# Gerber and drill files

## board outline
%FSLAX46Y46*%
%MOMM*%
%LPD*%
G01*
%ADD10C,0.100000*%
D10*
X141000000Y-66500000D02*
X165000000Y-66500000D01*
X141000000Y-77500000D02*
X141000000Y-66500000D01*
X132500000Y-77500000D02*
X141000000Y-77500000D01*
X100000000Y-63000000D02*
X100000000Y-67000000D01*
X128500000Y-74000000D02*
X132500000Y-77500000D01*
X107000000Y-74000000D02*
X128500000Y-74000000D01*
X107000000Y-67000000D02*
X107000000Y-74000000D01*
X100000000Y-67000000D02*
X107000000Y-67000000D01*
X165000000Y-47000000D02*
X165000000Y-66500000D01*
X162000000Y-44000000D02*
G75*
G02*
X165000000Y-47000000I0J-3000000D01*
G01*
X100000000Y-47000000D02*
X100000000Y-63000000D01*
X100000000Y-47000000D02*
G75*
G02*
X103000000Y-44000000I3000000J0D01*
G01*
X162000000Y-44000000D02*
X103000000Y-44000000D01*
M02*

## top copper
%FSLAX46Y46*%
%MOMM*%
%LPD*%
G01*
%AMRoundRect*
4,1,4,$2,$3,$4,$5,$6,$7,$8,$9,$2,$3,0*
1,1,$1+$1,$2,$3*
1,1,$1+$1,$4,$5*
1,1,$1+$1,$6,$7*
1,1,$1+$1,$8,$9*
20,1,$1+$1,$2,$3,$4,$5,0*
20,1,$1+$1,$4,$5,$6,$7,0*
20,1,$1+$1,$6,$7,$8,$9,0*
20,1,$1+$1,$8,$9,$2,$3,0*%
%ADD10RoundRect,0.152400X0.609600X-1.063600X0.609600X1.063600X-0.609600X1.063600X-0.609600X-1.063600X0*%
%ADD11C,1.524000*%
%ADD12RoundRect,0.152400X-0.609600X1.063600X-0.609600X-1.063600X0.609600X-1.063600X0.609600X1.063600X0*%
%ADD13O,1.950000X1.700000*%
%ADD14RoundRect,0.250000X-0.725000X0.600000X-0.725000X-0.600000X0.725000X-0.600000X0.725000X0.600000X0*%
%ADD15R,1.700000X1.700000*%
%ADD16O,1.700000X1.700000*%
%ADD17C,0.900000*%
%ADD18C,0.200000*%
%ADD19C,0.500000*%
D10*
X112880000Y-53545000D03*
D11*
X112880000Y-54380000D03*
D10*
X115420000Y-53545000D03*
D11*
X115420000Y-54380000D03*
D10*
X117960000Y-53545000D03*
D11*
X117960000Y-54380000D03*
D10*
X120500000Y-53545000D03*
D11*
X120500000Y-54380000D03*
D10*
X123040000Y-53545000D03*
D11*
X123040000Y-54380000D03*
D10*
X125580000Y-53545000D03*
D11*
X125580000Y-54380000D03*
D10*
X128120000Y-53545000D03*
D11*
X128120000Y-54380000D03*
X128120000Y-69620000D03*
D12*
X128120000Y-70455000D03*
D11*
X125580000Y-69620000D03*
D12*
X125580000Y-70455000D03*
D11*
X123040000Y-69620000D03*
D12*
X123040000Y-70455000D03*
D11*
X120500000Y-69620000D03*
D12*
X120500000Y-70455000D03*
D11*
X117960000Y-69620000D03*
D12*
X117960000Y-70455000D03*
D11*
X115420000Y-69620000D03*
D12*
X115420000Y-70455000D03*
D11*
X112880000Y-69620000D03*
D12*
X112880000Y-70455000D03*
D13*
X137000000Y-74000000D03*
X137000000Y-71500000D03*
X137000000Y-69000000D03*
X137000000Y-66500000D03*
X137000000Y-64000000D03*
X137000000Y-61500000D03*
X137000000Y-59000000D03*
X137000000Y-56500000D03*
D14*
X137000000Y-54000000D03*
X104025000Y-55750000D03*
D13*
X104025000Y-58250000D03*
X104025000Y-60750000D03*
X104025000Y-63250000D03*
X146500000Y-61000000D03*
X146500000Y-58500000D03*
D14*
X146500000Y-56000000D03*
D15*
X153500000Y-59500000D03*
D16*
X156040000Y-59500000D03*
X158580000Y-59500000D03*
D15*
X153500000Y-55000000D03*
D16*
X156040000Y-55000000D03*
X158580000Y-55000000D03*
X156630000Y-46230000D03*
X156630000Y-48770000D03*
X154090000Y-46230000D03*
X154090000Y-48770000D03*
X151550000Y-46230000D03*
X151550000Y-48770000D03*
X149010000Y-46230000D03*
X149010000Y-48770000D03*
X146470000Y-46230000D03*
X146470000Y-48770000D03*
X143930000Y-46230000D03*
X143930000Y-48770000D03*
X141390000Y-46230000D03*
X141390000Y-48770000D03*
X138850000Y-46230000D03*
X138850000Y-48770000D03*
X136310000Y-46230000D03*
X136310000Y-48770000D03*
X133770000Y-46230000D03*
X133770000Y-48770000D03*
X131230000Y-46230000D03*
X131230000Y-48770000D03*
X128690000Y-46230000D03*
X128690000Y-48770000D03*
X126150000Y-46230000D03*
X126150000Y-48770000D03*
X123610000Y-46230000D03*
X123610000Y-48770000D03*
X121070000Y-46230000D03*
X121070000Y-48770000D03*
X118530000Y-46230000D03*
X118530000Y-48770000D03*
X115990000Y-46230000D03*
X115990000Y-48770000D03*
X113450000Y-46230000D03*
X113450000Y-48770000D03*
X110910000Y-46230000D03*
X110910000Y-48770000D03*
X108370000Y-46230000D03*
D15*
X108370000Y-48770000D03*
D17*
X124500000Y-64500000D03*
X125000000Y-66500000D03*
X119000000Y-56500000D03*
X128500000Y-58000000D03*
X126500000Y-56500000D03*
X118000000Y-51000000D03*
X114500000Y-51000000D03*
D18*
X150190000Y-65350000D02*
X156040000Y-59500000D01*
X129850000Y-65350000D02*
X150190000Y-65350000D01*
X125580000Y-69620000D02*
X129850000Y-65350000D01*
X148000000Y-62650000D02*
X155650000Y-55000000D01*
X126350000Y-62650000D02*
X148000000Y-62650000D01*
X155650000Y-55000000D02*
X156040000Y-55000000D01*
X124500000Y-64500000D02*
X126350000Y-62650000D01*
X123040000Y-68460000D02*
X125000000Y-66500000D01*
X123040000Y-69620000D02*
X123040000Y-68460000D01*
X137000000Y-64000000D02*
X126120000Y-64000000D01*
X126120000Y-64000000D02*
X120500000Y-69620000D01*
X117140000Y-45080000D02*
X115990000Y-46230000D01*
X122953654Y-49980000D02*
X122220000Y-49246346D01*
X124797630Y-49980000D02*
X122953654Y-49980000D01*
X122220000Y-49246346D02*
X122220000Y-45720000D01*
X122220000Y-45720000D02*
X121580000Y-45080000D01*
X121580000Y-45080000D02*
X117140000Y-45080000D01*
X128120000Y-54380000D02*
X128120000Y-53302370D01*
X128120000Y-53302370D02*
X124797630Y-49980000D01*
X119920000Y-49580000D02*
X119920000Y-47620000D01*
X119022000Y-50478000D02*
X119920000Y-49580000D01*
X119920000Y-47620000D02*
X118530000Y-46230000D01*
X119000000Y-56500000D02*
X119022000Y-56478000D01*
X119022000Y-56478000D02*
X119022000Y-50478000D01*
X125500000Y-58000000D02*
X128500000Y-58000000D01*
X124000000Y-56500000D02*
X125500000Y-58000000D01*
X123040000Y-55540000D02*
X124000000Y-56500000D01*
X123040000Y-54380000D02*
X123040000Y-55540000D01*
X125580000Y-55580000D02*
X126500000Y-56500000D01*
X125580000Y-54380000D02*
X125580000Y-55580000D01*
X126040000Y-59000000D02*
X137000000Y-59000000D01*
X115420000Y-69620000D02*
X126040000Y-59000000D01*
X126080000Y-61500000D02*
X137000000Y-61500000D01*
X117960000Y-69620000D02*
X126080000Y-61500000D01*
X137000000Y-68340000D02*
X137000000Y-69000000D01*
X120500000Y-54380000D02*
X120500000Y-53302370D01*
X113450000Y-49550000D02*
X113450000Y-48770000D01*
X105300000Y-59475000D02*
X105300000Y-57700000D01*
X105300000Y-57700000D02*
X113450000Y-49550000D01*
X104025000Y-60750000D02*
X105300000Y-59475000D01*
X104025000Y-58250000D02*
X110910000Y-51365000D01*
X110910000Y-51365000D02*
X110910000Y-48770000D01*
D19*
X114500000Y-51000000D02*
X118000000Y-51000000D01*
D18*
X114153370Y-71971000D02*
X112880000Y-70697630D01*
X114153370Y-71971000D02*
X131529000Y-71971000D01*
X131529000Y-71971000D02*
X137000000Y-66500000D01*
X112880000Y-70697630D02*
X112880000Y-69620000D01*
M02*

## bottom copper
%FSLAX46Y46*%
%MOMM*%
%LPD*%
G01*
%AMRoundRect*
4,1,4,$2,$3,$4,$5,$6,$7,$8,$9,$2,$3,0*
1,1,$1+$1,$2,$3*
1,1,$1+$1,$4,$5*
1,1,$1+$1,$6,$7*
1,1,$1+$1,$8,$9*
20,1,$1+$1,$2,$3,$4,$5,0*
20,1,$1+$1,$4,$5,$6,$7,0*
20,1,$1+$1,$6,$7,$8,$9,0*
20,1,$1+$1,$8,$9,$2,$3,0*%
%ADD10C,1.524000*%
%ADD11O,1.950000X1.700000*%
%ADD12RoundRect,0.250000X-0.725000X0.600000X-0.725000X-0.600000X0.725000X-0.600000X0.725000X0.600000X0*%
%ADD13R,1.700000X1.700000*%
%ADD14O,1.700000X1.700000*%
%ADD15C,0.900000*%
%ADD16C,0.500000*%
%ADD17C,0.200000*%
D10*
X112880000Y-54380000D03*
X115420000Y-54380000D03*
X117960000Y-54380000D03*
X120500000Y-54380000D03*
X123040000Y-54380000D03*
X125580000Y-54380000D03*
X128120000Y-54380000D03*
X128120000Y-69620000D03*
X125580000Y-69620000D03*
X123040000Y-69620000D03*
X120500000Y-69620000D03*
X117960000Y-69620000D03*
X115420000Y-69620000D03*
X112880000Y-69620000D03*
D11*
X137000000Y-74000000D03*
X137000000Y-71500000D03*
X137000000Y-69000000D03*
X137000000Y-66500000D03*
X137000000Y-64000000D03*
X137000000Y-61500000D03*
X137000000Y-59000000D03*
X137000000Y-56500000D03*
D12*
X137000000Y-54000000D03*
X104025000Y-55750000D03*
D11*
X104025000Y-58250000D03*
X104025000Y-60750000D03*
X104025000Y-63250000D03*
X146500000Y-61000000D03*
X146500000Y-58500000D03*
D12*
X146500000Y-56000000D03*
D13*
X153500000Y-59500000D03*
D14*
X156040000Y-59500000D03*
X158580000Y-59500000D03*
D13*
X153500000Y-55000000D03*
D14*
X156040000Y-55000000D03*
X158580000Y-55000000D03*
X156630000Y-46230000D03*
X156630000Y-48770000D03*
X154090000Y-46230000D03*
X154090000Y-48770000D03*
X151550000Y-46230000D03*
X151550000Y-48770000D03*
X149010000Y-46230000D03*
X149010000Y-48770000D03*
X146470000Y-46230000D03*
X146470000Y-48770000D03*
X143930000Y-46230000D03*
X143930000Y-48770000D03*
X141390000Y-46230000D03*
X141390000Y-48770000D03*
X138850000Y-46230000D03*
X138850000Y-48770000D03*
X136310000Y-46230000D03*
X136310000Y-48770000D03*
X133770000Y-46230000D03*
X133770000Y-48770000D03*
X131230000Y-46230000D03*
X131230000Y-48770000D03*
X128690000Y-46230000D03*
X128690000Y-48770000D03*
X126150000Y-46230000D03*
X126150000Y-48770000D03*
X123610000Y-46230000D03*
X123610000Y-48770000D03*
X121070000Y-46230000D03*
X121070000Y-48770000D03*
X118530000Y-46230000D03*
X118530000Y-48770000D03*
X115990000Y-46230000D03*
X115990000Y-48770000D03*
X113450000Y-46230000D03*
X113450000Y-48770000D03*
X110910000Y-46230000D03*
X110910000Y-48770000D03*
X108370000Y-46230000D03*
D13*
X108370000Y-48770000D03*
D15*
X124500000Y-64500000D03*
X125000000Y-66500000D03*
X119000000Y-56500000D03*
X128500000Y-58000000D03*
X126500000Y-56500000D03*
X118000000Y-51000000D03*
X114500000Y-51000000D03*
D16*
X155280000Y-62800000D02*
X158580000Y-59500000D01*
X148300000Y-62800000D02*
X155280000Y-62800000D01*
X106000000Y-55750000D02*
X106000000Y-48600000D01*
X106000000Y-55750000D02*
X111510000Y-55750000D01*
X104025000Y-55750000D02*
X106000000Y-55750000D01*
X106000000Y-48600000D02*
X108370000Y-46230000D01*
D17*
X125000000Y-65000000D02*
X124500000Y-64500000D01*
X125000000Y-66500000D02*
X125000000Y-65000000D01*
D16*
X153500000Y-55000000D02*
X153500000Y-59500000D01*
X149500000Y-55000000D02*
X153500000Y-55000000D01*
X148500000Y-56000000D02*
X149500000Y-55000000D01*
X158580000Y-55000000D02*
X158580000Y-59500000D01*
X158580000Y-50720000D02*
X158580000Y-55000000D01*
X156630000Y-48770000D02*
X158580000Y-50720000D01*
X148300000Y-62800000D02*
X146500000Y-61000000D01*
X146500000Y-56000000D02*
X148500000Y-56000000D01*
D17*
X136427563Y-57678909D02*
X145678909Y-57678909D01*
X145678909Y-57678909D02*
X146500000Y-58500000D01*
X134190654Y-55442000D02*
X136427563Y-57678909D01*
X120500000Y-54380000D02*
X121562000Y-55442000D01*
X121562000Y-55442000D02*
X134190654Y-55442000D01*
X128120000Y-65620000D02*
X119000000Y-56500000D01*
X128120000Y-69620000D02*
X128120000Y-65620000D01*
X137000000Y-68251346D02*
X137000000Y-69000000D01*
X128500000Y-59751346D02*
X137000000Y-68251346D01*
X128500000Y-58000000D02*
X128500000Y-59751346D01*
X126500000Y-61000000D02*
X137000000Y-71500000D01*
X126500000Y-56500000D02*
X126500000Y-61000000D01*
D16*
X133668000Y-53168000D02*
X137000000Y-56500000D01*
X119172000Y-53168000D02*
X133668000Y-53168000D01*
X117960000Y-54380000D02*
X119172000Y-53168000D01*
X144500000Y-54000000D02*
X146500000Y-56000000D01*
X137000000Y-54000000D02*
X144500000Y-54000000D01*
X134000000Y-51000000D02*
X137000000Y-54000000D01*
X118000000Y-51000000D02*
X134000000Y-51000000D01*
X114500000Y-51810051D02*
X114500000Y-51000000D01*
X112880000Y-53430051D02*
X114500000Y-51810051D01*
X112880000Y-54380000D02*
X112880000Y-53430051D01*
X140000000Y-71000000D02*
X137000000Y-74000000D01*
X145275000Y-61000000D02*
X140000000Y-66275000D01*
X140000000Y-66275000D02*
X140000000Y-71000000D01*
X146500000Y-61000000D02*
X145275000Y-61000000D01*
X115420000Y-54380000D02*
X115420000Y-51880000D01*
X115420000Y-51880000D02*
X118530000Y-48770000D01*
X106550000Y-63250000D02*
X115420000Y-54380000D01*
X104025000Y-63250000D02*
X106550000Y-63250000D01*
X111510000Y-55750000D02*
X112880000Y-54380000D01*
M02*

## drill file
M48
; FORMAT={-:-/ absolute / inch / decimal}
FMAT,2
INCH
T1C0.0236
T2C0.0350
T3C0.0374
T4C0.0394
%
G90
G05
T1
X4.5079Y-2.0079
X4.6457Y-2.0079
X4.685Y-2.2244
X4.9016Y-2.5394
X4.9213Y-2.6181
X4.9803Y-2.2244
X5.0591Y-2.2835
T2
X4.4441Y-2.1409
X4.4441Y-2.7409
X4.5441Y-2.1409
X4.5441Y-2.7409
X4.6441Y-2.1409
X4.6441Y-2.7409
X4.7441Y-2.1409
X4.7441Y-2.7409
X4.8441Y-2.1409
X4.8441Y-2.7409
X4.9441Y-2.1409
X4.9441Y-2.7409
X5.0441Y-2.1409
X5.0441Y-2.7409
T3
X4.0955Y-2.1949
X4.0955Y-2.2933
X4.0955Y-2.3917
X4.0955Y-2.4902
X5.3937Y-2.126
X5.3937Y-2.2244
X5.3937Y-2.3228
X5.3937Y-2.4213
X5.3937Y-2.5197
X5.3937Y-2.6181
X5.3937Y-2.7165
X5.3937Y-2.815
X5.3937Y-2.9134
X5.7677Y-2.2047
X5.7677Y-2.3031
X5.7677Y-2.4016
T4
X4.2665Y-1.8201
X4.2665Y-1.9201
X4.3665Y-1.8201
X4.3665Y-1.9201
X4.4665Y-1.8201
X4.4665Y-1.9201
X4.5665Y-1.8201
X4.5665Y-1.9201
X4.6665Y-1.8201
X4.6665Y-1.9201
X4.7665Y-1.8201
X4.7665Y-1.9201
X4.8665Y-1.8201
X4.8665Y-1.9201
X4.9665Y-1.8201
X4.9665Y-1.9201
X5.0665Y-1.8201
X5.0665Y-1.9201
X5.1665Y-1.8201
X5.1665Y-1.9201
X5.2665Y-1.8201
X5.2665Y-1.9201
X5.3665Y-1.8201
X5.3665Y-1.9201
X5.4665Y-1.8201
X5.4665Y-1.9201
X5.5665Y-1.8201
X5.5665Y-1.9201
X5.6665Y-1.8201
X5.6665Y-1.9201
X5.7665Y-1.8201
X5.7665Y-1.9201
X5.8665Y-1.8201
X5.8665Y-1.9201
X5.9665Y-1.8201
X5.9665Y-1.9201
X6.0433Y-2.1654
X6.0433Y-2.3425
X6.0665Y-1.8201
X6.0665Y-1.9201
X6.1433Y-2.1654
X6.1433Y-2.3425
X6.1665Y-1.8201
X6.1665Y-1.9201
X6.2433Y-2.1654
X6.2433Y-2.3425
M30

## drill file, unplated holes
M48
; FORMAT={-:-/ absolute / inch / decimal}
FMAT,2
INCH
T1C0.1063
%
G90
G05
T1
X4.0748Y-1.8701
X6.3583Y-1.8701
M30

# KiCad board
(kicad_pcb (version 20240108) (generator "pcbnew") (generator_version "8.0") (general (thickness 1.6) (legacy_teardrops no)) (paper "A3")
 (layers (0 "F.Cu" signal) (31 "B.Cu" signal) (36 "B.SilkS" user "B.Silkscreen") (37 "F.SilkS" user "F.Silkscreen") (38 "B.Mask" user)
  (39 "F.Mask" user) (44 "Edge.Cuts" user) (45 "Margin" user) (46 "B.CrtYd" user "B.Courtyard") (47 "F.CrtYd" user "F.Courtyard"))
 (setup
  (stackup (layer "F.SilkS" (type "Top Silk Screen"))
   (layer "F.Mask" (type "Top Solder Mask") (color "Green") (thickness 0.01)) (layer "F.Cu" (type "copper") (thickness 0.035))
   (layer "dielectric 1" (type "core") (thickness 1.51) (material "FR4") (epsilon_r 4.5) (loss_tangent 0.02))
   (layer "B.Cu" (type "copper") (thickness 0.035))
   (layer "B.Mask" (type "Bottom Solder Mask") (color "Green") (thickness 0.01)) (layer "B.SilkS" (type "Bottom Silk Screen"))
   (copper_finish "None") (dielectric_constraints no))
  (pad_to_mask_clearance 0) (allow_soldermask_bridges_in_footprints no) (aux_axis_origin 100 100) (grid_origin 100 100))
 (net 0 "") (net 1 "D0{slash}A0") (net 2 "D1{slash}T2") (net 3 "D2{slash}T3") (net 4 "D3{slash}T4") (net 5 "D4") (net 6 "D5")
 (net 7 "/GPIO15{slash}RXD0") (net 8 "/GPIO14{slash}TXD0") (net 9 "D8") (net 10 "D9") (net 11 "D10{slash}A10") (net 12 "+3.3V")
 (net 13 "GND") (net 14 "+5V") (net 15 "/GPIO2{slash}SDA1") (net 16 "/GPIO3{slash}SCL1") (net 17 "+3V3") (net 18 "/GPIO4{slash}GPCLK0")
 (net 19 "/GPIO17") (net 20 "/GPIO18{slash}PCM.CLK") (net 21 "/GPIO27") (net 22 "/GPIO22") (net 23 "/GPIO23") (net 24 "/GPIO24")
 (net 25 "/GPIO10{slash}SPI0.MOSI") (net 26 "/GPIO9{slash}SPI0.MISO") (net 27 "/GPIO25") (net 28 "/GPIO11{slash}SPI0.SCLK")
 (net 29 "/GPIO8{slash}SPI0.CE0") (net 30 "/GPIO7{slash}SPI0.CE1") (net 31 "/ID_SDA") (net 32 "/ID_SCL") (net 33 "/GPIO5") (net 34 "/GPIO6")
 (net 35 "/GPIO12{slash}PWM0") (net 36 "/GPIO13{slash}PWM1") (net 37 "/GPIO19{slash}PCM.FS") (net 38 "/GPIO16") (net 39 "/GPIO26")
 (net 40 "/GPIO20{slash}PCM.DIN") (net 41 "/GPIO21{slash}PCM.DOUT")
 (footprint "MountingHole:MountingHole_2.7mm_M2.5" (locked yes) (layer "F.Cu") (at 161.5 47.5)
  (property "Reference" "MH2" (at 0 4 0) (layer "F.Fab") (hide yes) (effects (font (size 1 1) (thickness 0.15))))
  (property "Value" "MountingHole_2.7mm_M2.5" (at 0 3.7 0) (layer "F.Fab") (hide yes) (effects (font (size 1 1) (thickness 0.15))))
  (pad "" np_thru_hole circle (at 0 0) (size 2.7 2.7) (drill 2.7) (layers "*.Cu" "*.Mask")))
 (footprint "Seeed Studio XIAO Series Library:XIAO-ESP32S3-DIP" (layer "F.Cu") (at 120.5 62 90)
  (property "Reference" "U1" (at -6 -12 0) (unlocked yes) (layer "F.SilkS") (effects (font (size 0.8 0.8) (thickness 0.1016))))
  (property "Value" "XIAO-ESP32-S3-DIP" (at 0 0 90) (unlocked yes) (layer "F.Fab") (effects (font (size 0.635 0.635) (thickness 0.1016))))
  (pad "1" smd roundrect (at -8.455 -7.62 270) (size 2.432 1.524) (layers "F.Cu" "F.Mask") (roundrect_rratio 0.1) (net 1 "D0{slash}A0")
   (thermal_bridge_angle 45))
  (pad "1" thru_hole circle (at -7.62 -7.62 270) (size 1.524 1.524) (drill 0.889) (layers "*.Cu" "*.Mask") (remove_unused_layers no)
   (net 1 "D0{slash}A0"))
  (pad "2" smd roundrect (at -8.455 -5.08 270) (size 2.432 1.524) (layers "F.Cu" "F.Mask") (roundrect_rratio 0.1) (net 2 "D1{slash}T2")
   (thermal_bridge_angle 45))
  (pad "2" thru_hole circle (at -7.62 -5.08 270) (size 1.524 1.524) (drill 0.889) (layers "*.Cu" "*.Mask") (remove_unused_layers no)
   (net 2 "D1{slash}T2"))
  (pad "3" smd roundrect (at -8.455 -2.54 270) (size 2.432 1.524) (layers "F.Cu" "F.Mask") (roundrect_rratio 0.1) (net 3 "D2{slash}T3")
   (thermal_bridge_angle 45))
  (pad "3" thru_hole circle (at -7.62 -2.54 270) (size 1.524 1.524) (drill 0.889) (layers "*.Cu" "*.Mask") (remove_unused_layers no)
   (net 3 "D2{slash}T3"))
  (pad "4" smd roundrect (at -8.455 0 270) (size 2.432 1.524) (layers "F.Cu" "F.Mask") (roundrect_rratio 0.1) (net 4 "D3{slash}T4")
   (thermal_bridge_angle 45))
  (pad "4" thru_hole circle (at -7.62 0 270) (size 1.524 1.524) (drill 0.889) (layers "*.Cu" "*.Mask") (remove_unused_layers no)
   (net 4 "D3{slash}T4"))
  (pad "5" smd roundrect (at -8.455 2.54 270) (size 2.432 1.524) (layers "F.Cu" "F.Mask") (roundrect_rratio 0.1) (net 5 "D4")
   (thermal_bridge_angle 45))
  (pad "5" thru_hole circle (at -7.62 2.54 270) (size 1.524 1.524) (drill 0.889) (layers "*.Cu" "*.Mask") (remove_unused_layers no)
   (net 5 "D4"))
  (pad "6" smd roundrect (at -8.455 5.08 270) (size 2.432 1.524) (layers "F.Cu" "F.Mask") (roundrect_rratio 0.1) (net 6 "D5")
   (thermal_bridge_angle 45))
  (pad "6" thru_hole circle (at -7.62 5.08 270) (size 1.524 1.524) (drill 0.889) (layers "*.Cu" "*.Mask") (remove_unused_layers no)
   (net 6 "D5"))
  (pad "7" smd roundrect (at -8.455 7.62 270) (size 2.432 1.524) (layers "F.Cu" "F.Mask") (roundrect_rratio 0.1)
   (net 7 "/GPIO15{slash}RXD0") (thermal_bridge_angle 45))
  (pad "7" thru_hole circle (at -7.62 7.62 270) (size 1.524 1.524) (drill 0.889) (layers "*.Cu" "*.Mask") (remove_unused_layers no)
   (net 7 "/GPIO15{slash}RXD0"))
  (pad "8" thru_hole circle (at 7.62 7.62 90) (size 1.524 1.524) (drill 0.889) (layers "*.Cu" "*.Mask") (remove_unused_layers no)
   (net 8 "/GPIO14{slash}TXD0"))
  (pad "8" smd roundrect (at 8.455 7.62 90) (size 2.432 1.524) (layers "F.Cu" "F.Mask") (roundrect_rratio 0.1) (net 8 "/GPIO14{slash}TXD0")
   (thermal_bridge_angle 45))
  (pad "9" thru_hole circle (at 7.62 5.08 90) (size 1.524 1.524) (drill 0.889) (layers "*.Cu" "*.Mask") (remove_unused_layers no)
   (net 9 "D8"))
  (pad "9" smd roundrect (at 8.455 5.08 90) (size 2.432 1.524) (layers "F.Cu" "F.Mask") (roundrect_rratio 0.1) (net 9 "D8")
   (thermal_bridge_angle 45))
  (pad "10" thru_hole circle (at 7.62 2.54 90) (size 1.524 1.524) (drill 0.889) (layers "*.Cu" "*.Mask") (remove_unused_layers no)
   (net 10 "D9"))
  (pad "10" smd roundrect (at 8.455 2.54 90) (size 2.432 1.524) (layers "F.Cu" "F.Mask") (roundrect_rratio 0.1) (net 10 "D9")
   (thermal_bridge_angle 45))
  (pad "11" thru_hole circle (at 7.62 0 90) (size 1.524 1.524) (drill 0.889) (layers "*.Cu" "*.Mask") (remove_unused_layers no)
   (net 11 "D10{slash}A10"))
  (pad "11" smd roundrect (at 8.455 0 90) (size 2.432 1.524) (layers "F.Cu" "F.Mask") (roundrect_rratio 0.1) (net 11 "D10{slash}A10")
   (thermal_bridge_angle 45))
  (pad "12" thru_hole circle (at 7.62 -2.54 90) (size 1.524 1.524) (drill 0.889) (layers "*.Cu" "*.Mask") (remove_unused_layers no)
   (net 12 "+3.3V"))
  (pad "12" smd roundrect (at 8.455 -2.54 90) (size 2.432 1.524) (layers "F.Cu" "F.Mask") (roundrect_rratio 0.1) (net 12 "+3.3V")
   (thermal_bridge_angle 45))
  (pad "13" thru_hole circle (at 7.62 -5.08 90) (size 1.524 1.524) (drill 0.889) (layers "*.Cu" "*.Mask") (remove_unused_layers no)
   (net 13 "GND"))
  (pad "13" smd roundrect (at 8.455 -5.08 90) (size 2.432 1.524) (layers "F.Cu" "F.Mask") (roundrect_rratio 0.1) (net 13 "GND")
   (thermal_bridge_angle 45))
  (pad "14" thru_hole circle (at 7.62 -7.62 90) (size 1.524 1.524) (drill 0.889) (layers "*.Cu" "*.Mask") (remove_unused_layers no)
   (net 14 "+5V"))
  (pad "14" smd roundrect (at 8.455 -7.62 90) (size 2.432 1.524) (layers "F.Cu" "F.Mask") (roundrect_rratio 0.1) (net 14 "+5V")
   (thermal_bridge_angle 45)))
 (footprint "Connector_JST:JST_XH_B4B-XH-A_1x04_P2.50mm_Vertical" (layer "F.Cu") (at 104.025 55.75 -90)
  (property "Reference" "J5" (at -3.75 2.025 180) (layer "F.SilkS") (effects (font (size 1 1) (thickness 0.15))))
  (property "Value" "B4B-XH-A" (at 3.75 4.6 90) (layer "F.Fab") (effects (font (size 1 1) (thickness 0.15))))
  (pad "1" thru_hole roundrect (at 0 0 270) (size 1.7 1.95) (drill 0.95) (layers "*.Cu" "*.Mask") (remove_unused_layers no)
   (roundrect_rratio 0.147059) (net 14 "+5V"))
  (pad "2" thru_hole oval (at 2.5 0 270) (size 1.7 1.95) (drill 0.95) (layers "*.Cu" "*.Mask") (remove_unused_layers no)
   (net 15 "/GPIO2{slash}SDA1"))
  (pad "3" thru_hole oval (at 5 0 270) (size 1.7 1.95) (drill 0.95) (layers "*.Cu" "*.Mask") (remove_unused_layers no)
   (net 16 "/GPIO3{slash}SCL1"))
  (pad "4" thru_hole oval (at 7.5 0 270) (size 1.7 1.95) (drill 0.95) (layers "*.Cu" "*.Mask") (remove_unused_layers no) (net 13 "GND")))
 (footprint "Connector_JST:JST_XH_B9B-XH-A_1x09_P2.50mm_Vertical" (layer "F.Cu") (at 137 54 -90)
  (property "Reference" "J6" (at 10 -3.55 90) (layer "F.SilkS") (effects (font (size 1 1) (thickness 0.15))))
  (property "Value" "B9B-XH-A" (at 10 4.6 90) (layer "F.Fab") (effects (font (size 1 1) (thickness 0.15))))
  (pad "1" thru_hole roundrect (at 0 0 270) (size 1.7 1.95) (drill 0.95) (layers "*.Cu" "*.Mask") (remove_unused_layers no)
   (roundrect_rratio 0.147059) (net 14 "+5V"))
  (pad "2" thru_hole oval (at 2.5 0 270) (size 1.7 1.95) (drill 0.95) (layers "*.Cu" "*.Mask") (remove_unused_layers no) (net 12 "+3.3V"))
  (pad "3" thru_hole oval (at 5 0 270) (size 1.7 1.95) (drill 0.95) (layers "*.Cu" "*.Mask") (remove_unused_layers no) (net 2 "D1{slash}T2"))
  (pad "4" thru_hole oval (at 7.5 0 270) (size 1.7 1.95) (drill 0.95) (layers "*.Cu" "*.Mask") (remove_unused_layers no)
   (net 3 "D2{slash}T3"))
  (pad "5" thru_hole oval (at 10 0 270) (size 1.7 1.95) (drill 0.95) (layers "*.Cu" "*.Mask") (remove_unused_layers no)
   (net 4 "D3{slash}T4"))
  (pad "6" thru_hole oval (at 12.5 0 270) (size 1.7 1.95) (drill 0.95) (layers "*.Cu" "*.Mask") (remove_unused_layers no)
   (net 1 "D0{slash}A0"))
  (pad "7" thru_hole oval (at 15 0 270) (size 1.7 1.95) (drill 0.95) (layers "*.Cu" "*.Mask") (remove_unused_layers no) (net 10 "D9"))
  (pad "8" thru_hole oval (at 17.5 0 270) (size 1.7 1.95) (drill 0.95) (layers "*.Cu" "*.Mask") (remove_unused_layers no) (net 9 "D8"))
  (pad "9" thru_hole oval (at 20 0 270) (size 1.7 1.95) (drill 0.95) (layers "*.Cu" "*.Mask") (remove_unused_layers no) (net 13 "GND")))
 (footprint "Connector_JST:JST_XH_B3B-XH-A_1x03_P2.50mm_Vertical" (layer "F.Cu") (at 146.5 56 -90)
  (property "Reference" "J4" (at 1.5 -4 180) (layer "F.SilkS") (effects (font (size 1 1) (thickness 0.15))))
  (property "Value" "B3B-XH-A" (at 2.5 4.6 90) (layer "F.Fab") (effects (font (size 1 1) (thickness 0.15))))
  (pad "1" thru_hole roundrect (at 0 0 270) (size 1.7 1.95) (drill 0.95) (layers "*.Cu" "*.Mask") (remove_unused_layers no)
   (roundrect_rratio 0.147059) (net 14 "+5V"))
  (pad "2" thru_hole oval (at 2.5 0 270) (size 1.7 1.95) (drill 0.95) (layers "*.Cu" "*.Mask") (remove_unused_layers no)
   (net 11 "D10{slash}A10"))
  (pad "3" thru_hole oval (at 5 0 270) (size 1.7 1.95) (drill 0.95) (layers "*.Cu" "*.Mask") (remove_unused_layers no) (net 13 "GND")))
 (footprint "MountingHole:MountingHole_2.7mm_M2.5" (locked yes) (layer "F.Cu") (at 103.5 47.5)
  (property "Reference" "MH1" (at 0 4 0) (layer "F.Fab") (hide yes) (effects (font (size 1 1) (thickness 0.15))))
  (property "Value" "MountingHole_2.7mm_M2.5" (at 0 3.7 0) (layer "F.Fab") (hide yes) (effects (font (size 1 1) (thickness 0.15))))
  (pad "" np_thru_hole circle (at 0 0) (size 2.7 2.7) (drill 2.7) (layers "*.Cu" "*.Mask")))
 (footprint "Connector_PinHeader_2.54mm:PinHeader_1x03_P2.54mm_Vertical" (layer "F.Cu") (at 153.5 55 90)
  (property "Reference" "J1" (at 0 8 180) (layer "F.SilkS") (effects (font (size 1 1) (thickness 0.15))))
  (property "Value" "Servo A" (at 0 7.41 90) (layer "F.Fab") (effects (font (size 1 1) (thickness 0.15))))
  (pad "1" thru_hole rect (at 0 0 90) (size 1.7 1.7) (drill 1) (layers "*.Cu" "*.Mask") (remove_unused_layers no) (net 14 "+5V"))
  (pad "2" thru_hole oval (at 0 2.54 90) (size 1.7 1.7) (drill 1) (layers "*.Cu" "*.Mask") (remove_unused_layers no) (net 5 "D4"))
  (pad "3" thru_hole oval (at 0 5.08 90) (size 1.7 1.7) (drill 1) (layers "*.Cu" "*.Mask") (remove_unused_layers no) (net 13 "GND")))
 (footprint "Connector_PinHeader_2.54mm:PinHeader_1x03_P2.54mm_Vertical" (layer "F.Cu") (at 153.5 59.5 90)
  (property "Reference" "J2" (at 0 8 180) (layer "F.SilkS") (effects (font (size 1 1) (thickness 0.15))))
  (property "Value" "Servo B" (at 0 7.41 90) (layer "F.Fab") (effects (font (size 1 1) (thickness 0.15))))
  (pad "1" thru_hole rect (at 0 0 90) (size 1.7 1.7) (drill 1) (layers "*.Cu" "*.Mask") (remove_unused_layers no) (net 14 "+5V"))
  (pad "2" thru_hole oval (at 0 2.54 90) (size 1.7 1.7) (drill 1) (layers "*.Cu" "*.Mask") (remove_unused_layers no) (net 6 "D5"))
  (pad "3" thru_hole oval (at 0 5.08 90) (size 1.7 1.7) (drill 1) (layers "*.Cu" "*.Mask") (remove_unused_layers no) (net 13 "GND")))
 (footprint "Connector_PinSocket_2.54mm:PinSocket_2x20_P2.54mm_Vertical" (layer "B.Cu") (at 108.37 48.77 -90)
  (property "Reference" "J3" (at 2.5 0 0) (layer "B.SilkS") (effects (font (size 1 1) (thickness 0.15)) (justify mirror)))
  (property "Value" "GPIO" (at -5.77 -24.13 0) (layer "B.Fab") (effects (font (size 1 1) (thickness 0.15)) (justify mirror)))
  (pad "1" thru_hole rect (at 0 0 270) (size 1.7 1.7) (drill 1) (layers "*.Cu" "*.Mask") (remove_unused_layers no) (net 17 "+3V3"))
  (pad "2" thru_hole oval (at -2.54 0 270) (size 1.7 1.7) (drill 1) (layers "*.Cu" "*.Mask") (remove_unused_layers no) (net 14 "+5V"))
  (pad "3" thru_hole oval (at 0 -2.54 270) (size 1.7 1.7) (drill 1) (layers "*.Cu" "*.Mask") (remove_unused_layers no)
   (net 15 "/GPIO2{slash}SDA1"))
  (pad "4" thru_hole oval (at -2.54 -2.54 270) (size 1.7 1.7) (drill 1) (layers "*.Cu" "*.Mask") (remove_unused_layers no) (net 14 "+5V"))
  (pad "5" thru_hole oval (at 0 -5.08 270) (size 1.7 1.7) (drill 1) (layers "*.Cu" "*.Mask") (remove_unused_layers no)
   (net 16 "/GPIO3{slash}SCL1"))
  (pad "6" thru_hole oval (at -2.54 -5.08 270) (size 1.7 1.7) (drill 1) (layers "*.Cu" "*.Mask") (remove_unused_layers no) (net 13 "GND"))
  (pad "7" thru_hole oval (at 0 -7.62 270) (size 1.7 1.7) (drill 1) (layers "*.Cu" "*.Mask") (remove_unused_layers no)
   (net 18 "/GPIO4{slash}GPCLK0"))
  (pad "8" thru_hole oval (at -2.54 -7.62 270) (size 1.7 1.7) (drill 1) (layers "*.Cu" "*.Mask") (remove_unused_layers no)
   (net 8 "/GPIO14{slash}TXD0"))
  (pad "9" thru_hole oval (at 0 -10.16 270) (size 1.7 1.7) (drill 1) (layers "*.Cu" "*.Mask") (remove_unused_layers no) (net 13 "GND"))
  (pad "10" thru_hole oval (at -2.54 -10.16 270) (size 1.7 1.7) (drill 1) (layers "*.Cu" "*.Mask") (remove_unused_layers no)
   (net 7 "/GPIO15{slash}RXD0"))
  (pad "11" thru_hole oval (at 0 -12.7 270) (size 1.7 1.7) (drill 1) (layers "*.Cu" "*.Mask") (remove_unused_layers no) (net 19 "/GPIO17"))
  (pad "12" thru_hole oval (at -2.54 -12.7 270) (size 1.7 1.7) (drill 1) (layers "*.Cu" "*.Mask") (remove_unused_layers no)
   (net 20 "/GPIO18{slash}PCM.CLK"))
  (pad "13" thru_hole oval (at 0 -15.24 270) (size 1.7 1.7) (drill 1) (layers "*.Cu" "*.Mask") (remove_unused_layers no) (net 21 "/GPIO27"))
  (pad "14" thru_hole oval (at -2.54 -15.24 270) (size 1.7 1.7) (drill 1) (layers "*.Cu" "*.Mask") (remove_unused_layers no) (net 13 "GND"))
  (pad "15" thru_hole oval (at 0 -17.78 270) (size 1.7 1.7) (drill 1) (layers "*.Cu" "*.Mask") (remove_unused_layers no) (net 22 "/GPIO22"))
  (pad "16" thru_hole oval (at -2.54 -17.78 270) (size 1.7 1.7) (drill 1) (layers "*.Cu" "*.Mask") (remove_unused_layers no)
   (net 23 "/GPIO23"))
  (pad "17" thru_hole oval (at 0 -20.32 270) (size 1.7 1.7) (drill 1) (layers "*.Cu" "*.Mask") (remove_unused_layers no) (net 17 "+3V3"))
  (pad "18" thru_hole oval (at -2.54 -20.32 270) (size 1.7 1.7) (drill 1) (layers "*.Cu" "*.Mask") (remove_unused_layers no)
   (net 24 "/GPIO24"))
  (pad "19" thru_hole oval (at 0 -22.86 270) (size 1.7 1.7) (drill 1) (layers "*.Cu" "*.Mask") (remove_unused_layers no)
   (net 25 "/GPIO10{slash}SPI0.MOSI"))
  (pad "20" thru_hole oval (at -2.54 -22.86 270) (size 1.7 1.7) (drill 1) (layers "*.Cu" "*.Mask") (remove_unused_layers no) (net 13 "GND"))
  (pad "21" thru_hole oval (at 0 -25.4 270) (size 1.7 1.7) (drill 1) (layers "*.Cu" "*.Mask") (remove_unused_layers no)
   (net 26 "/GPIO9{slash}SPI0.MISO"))
  (pad "22" thru_hole oval (at -2.54 -25.4 270) (size 1.7 1.7) (drill 1) (layers "*.Cu" "*.Mask") (remove_unused_layers no)
   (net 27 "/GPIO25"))
  (pad "23" thru_hole oval (at 0 -27.94 270) (size 1.7 1.7) (drill 1) (layers "*.Cu" "*.Mask") (remove_unused_layers no)
   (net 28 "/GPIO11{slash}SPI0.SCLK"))
  (pad "24" thru_hole oval (at -2.54 -27.94 270) (size 1.7 1.7) (drill 1) (layers "*.Cu" "*.Mask") (remove_unused_layers no)
   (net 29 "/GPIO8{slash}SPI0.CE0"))
  (pad "25" thru_hole oval (at 0 -30.48 270) (size 1.7 1.7) (drill 1) (layers "*.Cu" "*.Mask") (remove_unused_layers no) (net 13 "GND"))
  (pad "26" thru_hole oval (at -2.54 -30.48 270) (size 1.7 1.7) (drill 1) (layers "*.Cu" "*.Mask") (remove_unused_layers no)
   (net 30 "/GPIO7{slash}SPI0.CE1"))
  (pad "27" thru_hole oval (at 0 -33.02 270) (size 1.7 1.7) (drill 1) (layers "*.Cu" "*.Mask") (remove_unused_layers no) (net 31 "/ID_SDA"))
  (pad "28" thru_hole oval (at -2.54 -33.02 270) (size 1.7 1.7) (drill 1) (layers "*.Cu" "*.Mask") (remove_unused_layers no)
   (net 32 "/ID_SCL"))
  (pad "29" thru_hole oval (at 0 -35.56 270) (size 1.7 1.7) (drill 1) (layers "*.Cu" "*.Mask") (remove_unused_layers no) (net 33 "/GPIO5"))
  (pad "30" thru_hole oval (at -2.54 -35.56 270) (size 1.7 1.7) (drill 1) (layers "*.Cu" "*.Mask") (remove_unused_layers no) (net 13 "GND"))
  (pad "31" thru_hole oval (at 0 -38.1 270) (size 1.7 1.7) (drill 1) (layers "*.Cu" "*.Mask") (remove_unused_layers no) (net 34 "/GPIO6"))
  (pad "32" thru_hole oval (at -2.54 -38.1 270) (size 1.7 1.7) (drill 1) (layers "*.Cu" "*.Mask") (remove_unused_layers no)
   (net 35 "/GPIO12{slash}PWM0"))
  (pad "33" thru_hole oval (at 0 -40.64 270) (size 1.7 1.7) (drill 1) (layers "*.Cu" "*.Mask") (remove_unused_layers no)
   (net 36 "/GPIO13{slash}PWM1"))
  (pad "34" thru_hole oval (at -2.54 -40.64 270) (size 1.7 1.7) (drill 1) (layers "*.Cu" "*.Mask") (remove_unused_layers no) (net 13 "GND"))
  (pad "35" thru_hole oval (at 0 -43.18 270) (size 1.7 1.7) (drill 1) (layers "*.Cu" "*.Mask") (remove_unused_layers no)
   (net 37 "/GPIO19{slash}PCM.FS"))
  (pad "36" thru_hole oval (at -2.54 -43.18 270) (size 1.7 1.7) (drill 1) (layers "*.Cu" "*.Mask") (remove_unused_layers no)
   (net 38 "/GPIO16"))
  (pad "37" thru_hole oval (at 0 -45.72 270) (size 1.7 1.7) (drill 1) (layers "*.Cu" "*.Mask") (remove_unused_layers no) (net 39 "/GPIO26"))
  (pad "38" thru_hole oval (at -2.54 -45.72 270) (size 1.7 1.7) (drill 1) (layers "*.Cu" "*.Mask") (remove_unused_layers no)
   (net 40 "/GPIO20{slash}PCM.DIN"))
  (pad "39" thru_hole oval (at 0 -48.26 270) (size 1.7 1.7) (drill 1) (layers "*.Cu" "*.Mask") (remove_unused_layers no) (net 13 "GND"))
  (pad "40" thru_hole oval (at -2.54 -48.26 270) (size 1.7 1.7) (drill 1) (layers "*.Cu" "*.Mask") (remove_unused_layers no)
   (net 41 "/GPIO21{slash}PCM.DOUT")))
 (gr_arc (start 162 44) (mid 164.12132 44.87868) (end 165 47) (stroke (width 0.1) (type solid)) (layer "Edge.Cuts"))
 (gr_line (start 132.5 77.5) (end 141 77.5) (stroke (width 0.1) (type default)) (layer "Edge.Cuts"))
 (gr_line (start 100 47) (end 100 63) (stroke (width 0.1) (type solid)) (layer "Edge.Cuts"))
 (gr_line (start 165 47) (end 165 66.5) (stroke (width 0.1) (type default)) (layer "Edge.Cuts"))
 (gr_line (start 141 66.5) (end 165 66.5) (stroke (width 0.1) (type default)) (layer "Edge.Cuts"))
 (gr_line (start 128.5 74) (end 132.5 77.5) (stroke (width 0.1) (type default)) (layer "Edge.Cuts"))
 (gr_line (start 107 74) (end 128.5 74) (stroke (width 0.1) (type default)) (layer "Edge.Cuts"))
 (gr_line (start 100 63) (end 100 67) (stroke (width 0.1) (type default)) (layer "Edge.Cuts"))
 (gr_line (start 141 77.5) (end 141 66.5) (stroke (width 0.1) (type default)) (layer "Edge.Cuts"))
 (gr_line (start 100 67) (end 107 67) (stroke (width 0.1) (type default)) (layer "Edge.Cuts"))
 (gr_arc (start 100 47) (mid 100.87868 44.87868) (end 103 44) (stroke (width 0.1) (type solid)) (layer "Edge.Cuts"))
 (gr_line (start 107 67) (end 107 74) (stroke (width 0.1) (type default)) (layer "Edge.Cuts"))
 (gr_line (start 162 44) (end 103 44) (stroke (width 0.1) (type solid)) (layer "Edge.Cuts"))
 (segment (start 146.5 61) (end 145.275 61) (width 0.5) (layer "B.Cu") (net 13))
 (segment (start 104.025 63.25) (end 106.55 63.25) (width 0.5) (layer "B.Cu") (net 13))
 (segment (start 156.63 48.77) (end 158.58 50.72) (width 0.5) (layer "B.Cu") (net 13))
 (segment (start 155.28 62.8) (end 158.58 59.5) (width 0.5) (layer "B.Cu") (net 13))
 (segment (start 115.42 51.88) (end 118.53 48.77) (width 0.5) (layer "B.Cu") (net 13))
 (segment (start 140 71) (end 137 74) (width 0.5) (layer "B.Cu") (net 13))
 (segment (start 115.42 54.38) (end 115.42 51.88) (width 0.5) (layer "B.Cu") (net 13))
 (segment (start 158.58 50.72) (end 158.58 55) (width 0.5) (layer "B.Cu") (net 13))
 (segment (start 140 66.275) (end 140 71) (width 0.5) (layer "B.Cu") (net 13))
 (segment (start 145.275 61) (end 140 66.275) (width 0.5) (layer "B.Cu") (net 13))
 (segment (start 148.3 62.8) (end 146.5 61) (width 0.5) (layer "B.Cu") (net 13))
 (segment (start 158.58 55) (end 158.58 59.5) (width 0.5) (layer "B.Cu") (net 13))
 (segment (start 106.55 63.25) (end 115.42 54.38) (width 0.5) (layer "B.Cu") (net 13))
 (segment (start 148.3 62.8) (end 155.28 62.8) (width 0.5) (layer "B.Cu") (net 13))
 (segment (start 104.025 58.25) (end 110.91 51.365) (width 0.2) (layer "F.Cu") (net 15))
 (segment (start 110.91 51.365) (end 110.91 48.77) (width 0.2) (layer "F.Cu") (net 15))
 (segment (start 104.025 60.75) (end 105.3 59.475) (width 0.2) (layer "F.Cu") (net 16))
 (segment (start 105.3 57.7) (end 113.45 49.55) (width 0.2) (layer "F.Cu") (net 16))
 (segment (start 113.45 49.55) (end 113.45 48.77) (width 0.2) (layer "F.Cu") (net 16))
 (segment (start 105.3 59.475) (end 105.3 57.7) (width 0.2) (layer "F.Cu") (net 16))
 (segment (start 122.953654 49.98) (end 122.22 49.246346) (width 0.2) (layer "F.Cu") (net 8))
 (segment (start 128.12 54.38) (end 128.12 53.30237) (width 0.2) (layer "F.Cu") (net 8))
 (segment (start 122.22 49.246346) (end 122.22 45.72) (width 0.2) (layer "F.Cu") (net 8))
 (segment (start 122.22 45.72) (end 121.58 45.08) (width 0.2) (layer "F.Cu") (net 8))
 (segment (start 121.58 45.08) (end 117.14 45.08) (width 0.2) (layer "F.Cu") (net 8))
 (segment (start 124.79763 49.98) (end 122.953654 49.98) (width 0.2) (layer "F.Cu") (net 8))
 (segment (start 128.12 53.30237) (end 124.79763 49.98) (width 0.2) (layer "F.Cu") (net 8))
 (segment (start 117.14 45.08) (end 115.99 46.23) (width 0.2) (layer "F.Cu") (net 8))
 (segment (start 119.92 47.62) (end 118.53 46.23) (width 0.2) (layer "F.Cu") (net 7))
 (segment (start 119.022 56.478) (end 119.022 50.478) (width 0.2) (layer "F.Cu") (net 7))
 (segment (start 119.92 49.58) (end 119.92 47.62) (width 0.2) (layer "F.Cu") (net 7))
 (segment (start 119.022 50.478) (end 119.92 49.58) (width 0.2) (layer "F.Cu") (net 7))
 (segment (start 119 56.5) (end 119.022 56.478) (width 0.2) (layer "F.Cu") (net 7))
 (via (at 119 56.5) (size 0.9) (drill 0.6) (layers "F.Cu" "B.Cu") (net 7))
 (segment (start 128.12 69.62) (end 128.12 65.62) (width 0.2) (layer "B.Cu") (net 7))
 (segment (start 128.12 65.62) (end 119 56.5) (width 0.2) (layer "B.Cu") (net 7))
 (segment (start 114.5 51) (end 118 51) (width 0.5) (layer "F.Cu") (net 14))
 (via (at 118 51) (size 0.9) (drill 0.6) (layers "F.Cu" "B.Cu") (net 14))
 (via (at 114.5 51) (size 0.9) (drill 0.6) (layers "F.Cu" "B.Cu") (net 14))
 (segment (start 112.88 53.430051) (end 114.5 51.810051) (width 0.5) (layer "B.Cu") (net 14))
 (segment (start 114.5 51.810051) (end 114.5 51) (width 0.5) (layer "B.Cu") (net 14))
 (segment (start 118 51) (end 134 51) (width 0.5) (layer "B.Cu") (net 14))
 (segment (start 149.5 55) (end 153.5 55) (width 0.5) (layer "B.Cu") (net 14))
 (segment (start 104.025 55.75) (end 106 55.75) (width 0.5) (layer "B.Cu") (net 14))
 (segment (start 137 54) (end 144.5 54) (width 0.5) (layer "B.Cu") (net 14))
 (segment (start 153.5 55) (end 153.5 59.5) (width 0.5) (layer "B.Cu") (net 14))
 (segment (start 106 48.6) (end 108.37 46.23) (width 0.5) (layer "B.Cu") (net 14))
 (segment (start 144.5 54) (end 146.5 56) (width 0.5) (layer "B.Cu") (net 14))
 (segment (start 146.5 56) (end 148.5 56) (width 0.5) (layer "B.Cu") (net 14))
 (segment (start 148.5 56) (end 149.5 55) (width 0.5) (layer "B.Cu") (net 14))
 (segment (start 106 55.75) (end 106 48.6) (width 0.5) (layer "B.Cu") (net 14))
 (segment (start 134 51) (end 137 54) (width 0.5) (layer "B.Cu") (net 14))
 (segment (start 112.88 54.38) (end 112.88 53.430051) (width 0.5) (layer "B.Cu") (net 14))
 (segment (start 106 55.75) (end 111.51 55.75) (width 0.5) (layer "B.Cu") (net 14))
 (segment (start 111.51 55.75) (end 112.88 54.38) (width 0.5) (layer "B.Cu") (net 14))
 (segment (start 155.65 55) (end 156.04 55) (width 0.2) (layer "F.Cu") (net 5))
 (segment (start 126.35 62.65) (end 148 62.65) (width 0.2) (layer "F.Cu") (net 5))
 (segment (start 123.04 69.62) (end 123.04 68.46) (width 0.2) (layer "F.Cu") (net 5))
 (segment (start 124.5 64.5) (end 126.35 62.65) (width 0.2) (layer "F.Cu") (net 5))
 (segment (start 148 62.65) (end 155.65 55) (width 0.2) (layer "F.Cu") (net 5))
 (segment (start 123.04 68.46) (end 125 66.5) (width 0.2) (layer "F.Cu") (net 5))
 (via (at 124.5 64.5) (size 0.9) (drill 0.6) (layers "F.Cu" "B.Cu") (free yes) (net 5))
 (via (at 125 66.5) (size 0.9) (drill 0.6) (layers "F.Cu" "B.Cu") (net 5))
 (segment (start 125 65) (end 124.5 64.5) (width 0.2) (layer "B.Cu") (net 5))
 (segment (start 125 66.5) (end 125 65) (width 0.2) (layer "B.Cu") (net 5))
 (segment (start 129.85 65.35) (end 150.19 65.35) (width 0.2) (layer "F.Cu") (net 6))
 (segment (start 150.19 65.35) (end 156.04 59.5) (width 0.2) (layer "F.Cu") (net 6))
 (segment (start 125.58 69.62) (end 129.85 65.35) (width 0.2) (layer "F.Cu") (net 6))
 (segment (start 120.5 54.38) (end 120.5 53.30237) (width 0.2) (layer "F.Cu") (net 11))
 (segment (start 134.190654 55.442) (end 136.427563 57.678909) (width 0.2) (layer "B.Cu") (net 11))
 (segment (start 121.562 55.442) (end 134.190654 55.442) (width 0.2) (layer "B.Cu") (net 11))
 (segment (start 136.427563 57.678909) (end 145.678909 57.678909) (width 0.2) (layer "B.Cu") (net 11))
 (segment (start 145.678909 57.678909) (end 146.5 58.5) (width 0.2) (layer "B.Cu") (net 11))
 (segment (start 120.5 54.38) (end 121.562 55.442) (width 0.2) (layer "B.Cu") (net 11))
 (segment (start 137 64) (end 126.12 64) (width 0.2) (layer "F.Cu") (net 4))
 (segment (start 126.12 64) (end 120.5 69.62) (width 0.2) (layer "F.Cu") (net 4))
 (segment (start 112.88 70.69763) (end 112.88 69.62) (width 0.2) (layer "F.Cu") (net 1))
 (segment (start 114.15337 71.971) (end 131.529 71.971) (width 0.2) (layer "F.Cu") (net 1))
 (segment (start 131.529 71.971) (end 137 66.5) (width 0.2) (layer "F.Cu") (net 1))
 (segment (start 114.15337 71.971) (end 112.88 70.69763) (width 0.2) (layer "F.Cu") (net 1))
 (segment (start 117.96 69.62) (end 126.08 61.5) (width 0.2) (layer "F.Cu") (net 3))
 (segment (start 126.08 61.5) (end 137 61.5) (width 0.2) (layer "F.Cu") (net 3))
 (segment (start 123.04 55.54) (end 124 56.5) (width 0.2) (layer "F.Cu") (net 10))
 (segment (start 124 56.5) (end 125.5 58) (width 0.2) (layer "F.Cu") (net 10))
 (segment (start 123.04 54.38) (end 123.04 55.54) (width 0.2) (layer "F.Cu") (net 10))
 (segment (start 137 68.34) (end 137 69) (width 0.2) (layer "F.Cu") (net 10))
 (segment (start 125.5 58) (end 128.5 58) (width 0.2) (layer "F.Cu") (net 10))
 (via (at 128.5 58) (size 0.9) (drill 0.6) (layers "F.Cu" "B.Cu") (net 10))
 (segment (start 128.5 58) (end 128.5 59.751346) (width 0.2) (layer "B.Cu") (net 10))
 (segment (start 128.5 59.751346) (end 137 68.251346) (width 0.2) (layer "B.Cu") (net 10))
 (segment (start 137 68.251346) (end 137 69) (width 0.2) (layer "B.Cu") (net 10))
 (segment (start 126.04 59) (end 137 59) (width 0.2) (layer "F.Cu") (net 2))
 (segment (start 115.42 69.62) (end 126.04 59) (width 0.2) (layer "F.Cu") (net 2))
 (segment (start 125.58 55.58) (end 126.5 56.5) (width 0.2) (layer "F.Cu") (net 9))
 (segment (start 125.58 54.38) (end 125.58 55.58) (width 0.2) (layer "F.Cu") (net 9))
 (via (at 126.5 56.5) (size 0.9) (drill 0.6) (layers "F.Cu" "B.Cu") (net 9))
 (segment (start 126.5 61) (end 137 71.5) (width 0.2) (layer "B.Cu") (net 9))
 (segment (start 126.5 56.5) (end 126.5 61) (width 0.2) (layer "B.Cu") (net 9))
 (segment (start 119.172 53.168) (end 133.668 53.168) (width 0.5) (layer "B.Cu") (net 12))
 (segment (start 133.668 53.168) (end 137 56.5) (width 0.5) (layer "B.Cu") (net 12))
 (segment (start 117.96 54.38) (end 119.172 53.168) (width 0.5) (layer "B.Cu") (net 12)))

